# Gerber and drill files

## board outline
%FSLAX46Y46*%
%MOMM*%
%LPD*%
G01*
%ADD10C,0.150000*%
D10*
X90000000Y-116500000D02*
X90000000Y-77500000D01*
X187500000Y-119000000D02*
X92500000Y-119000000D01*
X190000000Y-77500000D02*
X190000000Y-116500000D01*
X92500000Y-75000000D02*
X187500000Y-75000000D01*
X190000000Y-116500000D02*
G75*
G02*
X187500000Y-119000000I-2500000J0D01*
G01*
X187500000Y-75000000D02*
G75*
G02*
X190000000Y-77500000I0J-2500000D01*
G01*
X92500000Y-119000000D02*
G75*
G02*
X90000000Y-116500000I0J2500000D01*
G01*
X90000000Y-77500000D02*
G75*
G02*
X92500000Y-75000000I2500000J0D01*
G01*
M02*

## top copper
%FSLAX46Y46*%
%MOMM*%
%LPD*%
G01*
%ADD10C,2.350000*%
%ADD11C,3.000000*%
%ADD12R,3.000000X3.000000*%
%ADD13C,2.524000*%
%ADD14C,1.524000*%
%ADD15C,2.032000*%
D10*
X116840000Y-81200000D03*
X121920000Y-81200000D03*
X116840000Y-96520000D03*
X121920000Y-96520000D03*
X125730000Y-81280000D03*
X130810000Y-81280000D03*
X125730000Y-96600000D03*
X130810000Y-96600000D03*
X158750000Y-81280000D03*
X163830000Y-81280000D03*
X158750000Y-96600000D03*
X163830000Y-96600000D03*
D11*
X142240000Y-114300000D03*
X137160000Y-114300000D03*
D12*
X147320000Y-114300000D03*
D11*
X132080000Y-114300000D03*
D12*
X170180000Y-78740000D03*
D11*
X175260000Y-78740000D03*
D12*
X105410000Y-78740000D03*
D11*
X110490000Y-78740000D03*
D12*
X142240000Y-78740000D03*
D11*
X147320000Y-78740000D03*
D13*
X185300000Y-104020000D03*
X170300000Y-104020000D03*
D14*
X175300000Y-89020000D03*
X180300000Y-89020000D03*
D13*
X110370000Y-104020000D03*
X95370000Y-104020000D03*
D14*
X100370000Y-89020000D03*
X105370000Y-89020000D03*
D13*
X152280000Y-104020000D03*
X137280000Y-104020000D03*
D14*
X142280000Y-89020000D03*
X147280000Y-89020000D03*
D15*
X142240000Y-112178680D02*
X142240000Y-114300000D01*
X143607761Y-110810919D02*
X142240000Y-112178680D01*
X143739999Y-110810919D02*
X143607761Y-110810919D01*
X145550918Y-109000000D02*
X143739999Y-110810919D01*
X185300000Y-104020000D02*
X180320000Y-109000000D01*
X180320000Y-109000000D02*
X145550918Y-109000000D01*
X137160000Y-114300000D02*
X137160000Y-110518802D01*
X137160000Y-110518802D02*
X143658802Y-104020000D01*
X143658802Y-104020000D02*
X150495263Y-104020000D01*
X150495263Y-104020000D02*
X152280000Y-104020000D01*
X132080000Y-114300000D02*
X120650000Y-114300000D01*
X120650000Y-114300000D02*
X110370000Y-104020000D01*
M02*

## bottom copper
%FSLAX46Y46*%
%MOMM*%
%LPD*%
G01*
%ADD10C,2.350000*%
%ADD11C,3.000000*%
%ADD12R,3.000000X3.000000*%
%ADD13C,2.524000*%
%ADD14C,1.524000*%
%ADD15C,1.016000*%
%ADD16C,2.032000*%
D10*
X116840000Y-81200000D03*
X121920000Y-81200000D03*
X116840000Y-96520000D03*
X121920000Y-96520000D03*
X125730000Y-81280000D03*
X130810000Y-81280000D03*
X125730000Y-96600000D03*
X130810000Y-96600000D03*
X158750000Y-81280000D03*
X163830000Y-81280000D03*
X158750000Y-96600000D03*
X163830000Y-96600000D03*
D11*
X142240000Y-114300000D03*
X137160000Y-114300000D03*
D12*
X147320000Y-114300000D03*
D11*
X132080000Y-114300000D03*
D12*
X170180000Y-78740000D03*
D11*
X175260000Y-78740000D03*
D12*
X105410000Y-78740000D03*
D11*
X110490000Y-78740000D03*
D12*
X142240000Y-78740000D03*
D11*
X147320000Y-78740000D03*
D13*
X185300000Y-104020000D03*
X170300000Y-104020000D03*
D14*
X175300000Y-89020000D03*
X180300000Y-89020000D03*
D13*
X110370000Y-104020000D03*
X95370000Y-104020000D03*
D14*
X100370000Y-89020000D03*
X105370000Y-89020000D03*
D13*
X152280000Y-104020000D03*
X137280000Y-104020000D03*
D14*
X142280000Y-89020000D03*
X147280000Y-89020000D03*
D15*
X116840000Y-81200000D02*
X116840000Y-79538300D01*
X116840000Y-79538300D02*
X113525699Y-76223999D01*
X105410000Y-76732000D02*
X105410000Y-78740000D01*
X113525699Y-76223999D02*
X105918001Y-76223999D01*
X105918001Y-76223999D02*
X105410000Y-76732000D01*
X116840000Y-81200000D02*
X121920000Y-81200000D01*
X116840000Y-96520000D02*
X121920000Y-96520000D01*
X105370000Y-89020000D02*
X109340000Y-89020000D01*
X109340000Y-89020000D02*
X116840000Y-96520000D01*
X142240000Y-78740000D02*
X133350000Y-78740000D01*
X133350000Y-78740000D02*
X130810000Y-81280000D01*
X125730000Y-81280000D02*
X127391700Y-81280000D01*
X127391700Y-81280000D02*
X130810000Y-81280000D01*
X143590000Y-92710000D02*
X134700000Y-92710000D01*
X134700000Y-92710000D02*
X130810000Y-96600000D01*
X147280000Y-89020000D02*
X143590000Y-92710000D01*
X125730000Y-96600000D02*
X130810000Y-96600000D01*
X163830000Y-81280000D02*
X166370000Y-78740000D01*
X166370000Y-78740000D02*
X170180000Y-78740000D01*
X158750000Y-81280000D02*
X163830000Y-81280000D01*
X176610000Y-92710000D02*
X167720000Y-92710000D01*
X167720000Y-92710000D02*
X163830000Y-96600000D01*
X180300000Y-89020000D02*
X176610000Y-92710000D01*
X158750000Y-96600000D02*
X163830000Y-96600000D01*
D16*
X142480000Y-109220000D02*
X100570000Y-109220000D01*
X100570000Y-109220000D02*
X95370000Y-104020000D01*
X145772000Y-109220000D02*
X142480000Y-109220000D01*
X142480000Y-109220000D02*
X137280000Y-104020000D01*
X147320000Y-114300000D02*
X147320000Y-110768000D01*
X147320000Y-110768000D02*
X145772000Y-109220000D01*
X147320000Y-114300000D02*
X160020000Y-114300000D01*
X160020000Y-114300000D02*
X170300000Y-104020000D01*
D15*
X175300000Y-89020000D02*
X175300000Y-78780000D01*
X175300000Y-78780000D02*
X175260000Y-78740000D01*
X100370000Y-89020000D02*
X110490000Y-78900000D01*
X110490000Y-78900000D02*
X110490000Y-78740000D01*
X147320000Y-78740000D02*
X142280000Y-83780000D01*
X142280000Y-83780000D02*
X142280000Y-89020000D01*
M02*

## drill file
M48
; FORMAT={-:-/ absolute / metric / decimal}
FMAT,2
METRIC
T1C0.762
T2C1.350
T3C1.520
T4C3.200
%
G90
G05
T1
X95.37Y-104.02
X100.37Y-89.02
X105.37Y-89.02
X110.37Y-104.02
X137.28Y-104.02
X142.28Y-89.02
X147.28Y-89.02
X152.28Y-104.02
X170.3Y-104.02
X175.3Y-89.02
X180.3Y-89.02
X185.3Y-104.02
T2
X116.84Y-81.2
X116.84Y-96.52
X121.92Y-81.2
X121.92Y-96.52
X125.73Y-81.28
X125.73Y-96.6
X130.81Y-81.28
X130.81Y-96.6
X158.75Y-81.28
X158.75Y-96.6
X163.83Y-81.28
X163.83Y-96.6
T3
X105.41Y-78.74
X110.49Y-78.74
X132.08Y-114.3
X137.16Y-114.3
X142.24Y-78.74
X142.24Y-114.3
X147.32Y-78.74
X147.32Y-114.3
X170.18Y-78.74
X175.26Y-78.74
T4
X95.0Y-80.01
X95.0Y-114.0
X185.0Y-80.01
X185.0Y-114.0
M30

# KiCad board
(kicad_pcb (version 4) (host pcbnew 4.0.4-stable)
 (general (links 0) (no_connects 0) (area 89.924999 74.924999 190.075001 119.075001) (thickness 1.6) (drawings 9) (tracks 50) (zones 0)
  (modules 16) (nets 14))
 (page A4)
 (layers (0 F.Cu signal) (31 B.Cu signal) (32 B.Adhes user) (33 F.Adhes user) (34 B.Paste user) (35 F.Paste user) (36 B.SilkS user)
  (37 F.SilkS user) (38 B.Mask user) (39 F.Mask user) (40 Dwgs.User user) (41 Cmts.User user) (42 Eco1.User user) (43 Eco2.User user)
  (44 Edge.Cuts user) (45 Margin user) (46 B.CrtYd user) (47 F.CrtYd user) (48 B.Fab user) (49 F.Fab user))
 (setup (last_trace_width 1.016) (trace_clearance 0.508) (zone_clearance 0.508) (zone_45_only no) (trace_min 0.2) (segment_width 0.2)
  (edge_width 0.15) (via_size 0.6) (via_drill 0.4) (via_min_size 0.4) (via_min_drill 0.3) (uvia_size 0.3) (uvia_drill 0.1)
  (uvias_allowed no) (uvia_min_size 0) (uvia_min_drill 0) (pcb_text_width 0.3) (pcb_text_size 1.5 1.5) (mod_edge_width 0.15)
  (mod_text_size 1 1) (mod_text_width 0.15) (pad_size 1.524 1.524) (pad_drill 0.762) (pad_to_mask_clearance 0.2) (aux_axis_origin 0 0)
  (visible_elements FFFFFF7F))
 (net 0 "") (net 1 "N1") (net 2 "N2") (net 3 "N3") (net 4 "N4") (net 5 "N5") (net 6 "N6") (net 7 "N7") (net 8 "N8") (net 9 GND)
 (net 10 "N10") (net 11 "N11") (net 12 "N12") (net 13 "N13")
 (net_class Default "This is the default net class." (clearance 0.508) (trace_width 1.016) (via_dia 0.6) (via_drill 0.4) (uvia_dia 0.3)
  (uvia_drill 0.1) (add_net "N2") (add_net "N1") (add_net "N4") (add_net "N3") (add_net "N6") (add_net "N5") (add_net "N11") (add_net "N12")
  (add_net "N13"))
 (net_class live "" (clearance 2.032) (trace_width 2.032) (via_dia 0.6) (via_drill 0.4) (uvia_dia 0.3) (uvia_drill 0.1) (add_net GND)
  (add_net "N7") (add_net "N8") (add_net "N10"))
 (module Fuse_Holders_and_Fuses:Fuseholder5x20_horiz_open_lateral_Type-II (layer F.Cu) (at 116.84 96.52 90)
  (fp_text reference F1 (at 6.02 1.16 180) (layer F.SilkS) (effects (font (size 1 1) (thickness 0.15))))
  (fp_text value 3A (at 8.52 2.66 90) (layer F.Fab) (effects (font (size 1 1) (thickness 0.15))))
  (pad 2 thru_hole circle (at 15.32 0 90) (size 2.35 2.35) (drill 1.35) (layers *.Cu *.Mask) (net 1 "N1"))
  (pad 2 thru_hole circle (at 15.32 5.08 90) (size 2.35 2.35) (drill 1.35) (layers *.Cu *.Mask) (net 1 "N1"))
  (pad 1 thru_hole circle (at 0 0 90) (size 2.35 2.35) (drill 1.35) (layers *.Cu *.Mask) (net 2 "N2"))
  (pad 1 thru_hole circle (at 0 5.08 90) (size 2.35 2.35) (drill 1.35) (layers *.Cu *.Mask) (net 2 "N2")))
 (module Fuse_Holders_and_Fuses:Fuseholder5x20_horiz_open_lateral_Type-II (layer F.Cu) (at 125.73 96.6 90)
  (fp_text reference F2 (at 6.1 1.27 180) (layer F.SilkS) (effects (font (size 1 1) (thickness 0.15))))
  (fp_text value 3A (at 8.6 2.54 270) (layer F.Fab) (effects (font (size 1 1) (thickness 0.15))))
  (pad 2 thru_hole circle (at 15.32 0 90) (size 2.35 2.35) (drill 1.35) (layers *.Cu *.Mask) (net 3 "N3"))
  (pad 2 thru_hole circle (at 15.32 5.08 90) (size 2.35 2.35) (drill 1.35) (layers *.Cu *.Mask) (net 3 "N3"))
  (pad 1 thru_hole circle (at 0 0 90) (size 2.35 2.35) (drill 1.35) (layers *.Cu *.Mask) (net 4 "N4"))
  (pad 1 thru_hole circle (at 0 5.08 90) (size 2.35 2.35) (drill 1.35) (layers *.Cu *.Mask) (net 4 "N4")))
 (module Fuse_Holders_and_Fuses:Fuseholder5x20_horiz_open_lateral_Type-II (layer F.Cu) (at 158.75 96.6 90)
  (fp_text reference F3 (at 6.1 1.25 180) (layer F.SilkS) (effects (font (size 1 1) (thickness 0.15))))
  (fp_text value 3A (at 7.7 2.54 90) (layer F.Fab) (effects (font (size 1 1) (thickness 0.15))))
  (pad 2 thru_hole circle (at 15.32 0 90) (size 2.35 2.35) (drill 1.35) (layers *.Cu *.Mask) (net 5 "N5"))
  (pad 2 thru_hole circle (at 15.32 5.08 90) (size 2.35 2.35) (drill 1.35) (layers *.Cu *.Mask) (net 5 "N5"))
  (pad 1 thru_hole circle (at 0 0 90) (size 2.35 2.35) (drill 1.35) (layers *.Cu *.Mask) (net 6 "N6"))
  (pad 1 thru_hole circle (at 0 5.08 90) (size 2.35 2.35) (drill 1.35) (layers *.Cu *.Mask) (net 6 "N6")))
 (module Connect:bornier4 (layer F.Cu) (at 147.32 114.3 180)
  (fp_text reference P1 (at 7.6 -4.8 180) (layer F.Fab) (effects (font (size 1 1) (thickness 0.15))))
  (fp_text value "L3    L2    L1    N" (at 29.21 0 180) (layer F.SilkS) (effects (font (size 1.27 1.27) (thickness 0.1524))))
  (pad 2 thru_hole circle (at 5.08 0 180) (size 3 3) (drill 1.52) (layers *.Cu *.Mask) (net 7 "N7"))
  (pad 3 thru_hole circle (at 10.16 0 180) (size 3 3) (drill 1.52) (layers *.Cu *.Mask) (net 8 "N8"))
  (pad 1 thru_hole rect (at 0 0 180) (size 3 3) (drill 1.52) (layers *.Cu *.Mask) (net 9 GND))
  (pad 4 thru_hole circle (at 15.24 0 180) (size 3 3) (drill 1.52) (layers *.Cu *.Mask) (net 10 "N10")))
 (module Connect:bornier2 (layer F.Cu) (at 170.18 78.74)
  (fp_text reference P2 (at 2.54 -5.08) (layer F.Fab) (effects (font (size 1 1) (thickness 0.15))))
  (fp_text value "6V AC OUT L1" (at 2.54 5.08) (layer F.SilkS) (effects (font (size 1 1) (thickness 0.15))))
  (pad 1 thru_hole rect (at 0 0) (size 3 3) (drill 1.52) (layers *.Cu *.Mask) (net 5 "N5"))
  (pad 2 thru_hole circle (at 5.08 0) (size 3 3) (drill 1.52) (layers *.Cu *.Mask) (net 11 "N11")))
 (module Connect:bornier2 (layer F.Cu) (at 105.41 78.74)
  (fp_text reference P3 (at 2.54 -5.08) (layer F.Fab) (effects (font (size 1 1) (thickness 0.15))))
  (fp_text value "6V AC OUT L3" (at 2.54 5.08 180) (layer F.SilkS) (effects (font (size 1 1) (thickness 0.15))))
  (pad 1 thru_hole rect (at 0 0) (size 3 3) (drill 1.52) (layers *.Cu *.Mask) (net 1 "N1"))
  (pad 2 thru_hole circle (at 5.08 0) (size 3 3) (drill 1.52) (layers *.Cu *.Mask) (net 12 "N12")))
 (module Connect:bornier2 (layer F.Cu) (at 142.24 78.74)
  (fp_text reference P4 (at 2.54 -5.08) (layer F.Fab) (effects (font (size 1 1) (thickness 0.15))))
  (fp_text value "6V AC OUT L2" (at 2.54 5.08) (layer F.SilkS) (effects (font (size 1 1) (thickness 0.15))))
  (pad 1 thru_hole rect (at 0 0) (size 3 3) (drill 1.52) (layers *.Cu *.Mask) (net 3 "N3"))
  (pad 2 thru_hole circle (at 5.08 0) (size 3 3) (drill 1.52) (layers *.Cu *.Mask) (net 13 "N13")))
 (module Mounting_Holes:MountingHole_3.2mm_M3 (layer F.Cu) (at 185 80.01 90)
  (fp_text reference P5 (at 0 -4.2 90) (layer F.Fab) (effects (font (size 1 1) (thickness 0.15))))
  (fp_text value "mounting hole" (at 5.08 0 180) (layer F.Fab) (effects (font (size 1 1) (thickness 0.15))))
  (pad 1 np_thru_hole circle (at 0 0 90) (size 3.2 3.2) (drill 3.2) (layers *.Cu *.Mask)))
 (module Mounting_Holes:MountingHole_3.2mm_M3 (layer F.Cu) (at 185 114 90)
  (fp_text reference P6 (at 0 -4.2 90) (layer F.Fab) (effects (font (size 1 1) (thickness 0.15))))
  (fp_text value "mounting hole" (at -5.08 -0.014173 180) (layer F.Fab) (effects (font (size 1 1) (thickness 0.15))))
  (pad 1 np_thru_hole circle (at 0 0 90) (size 3.2 3.2) (drill 3.2) (layers *.Cu *.Mask)))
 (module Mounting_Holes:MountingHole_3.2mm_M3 (layer F.Cu) (at 95 114 90)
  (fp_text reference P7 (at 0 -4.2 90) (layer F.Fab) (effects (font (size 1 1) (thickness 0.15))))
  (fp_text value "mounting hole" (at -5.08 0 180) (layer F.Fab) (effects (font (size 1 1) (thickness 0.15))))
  (pad 1 np_thru_hole circle (at 0 0 90) (size 3.2 3.2) (drill 3.2) (layers *.Cu *.Mask)))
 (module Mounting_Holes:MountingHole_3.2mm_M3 (layer F.Cu) (at 95 80.01 90)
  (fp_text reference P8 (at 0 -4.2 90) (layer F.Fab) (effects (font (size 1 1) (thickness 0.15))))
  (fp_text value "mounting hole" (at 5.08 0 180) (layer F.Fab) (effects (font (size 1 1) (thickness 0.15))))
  (pad 1 np_thru_hole circle (at 0 0 90) (size 3.2 3.2) (drill 3.2) (layers *.Cu *.Mask)))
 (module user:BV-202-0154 (layer F.Cu) (at 177.8 96.52 90)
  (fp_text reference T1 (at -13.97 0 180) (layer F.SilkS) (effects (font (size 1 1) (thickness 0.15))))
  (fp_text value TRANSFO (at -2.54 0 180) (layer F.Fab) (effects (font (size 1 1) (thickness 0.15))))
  (pad 1 thru_hole circle (at -7.5 7.5 90) (size 2.524 2.524) (drill 0.762) (layers *.Cu *.Mask) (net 7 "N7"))
  (pad 2 thru_hole circle (at -7.5 -7.5 90) (size 2.524 2.524) (drill 0.762) (layers *.Cu *.Mask) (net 9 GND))
  (pad 3 thru_hole circle (at 7.5 -2.5 90) (size 1.524 1.524) (drill 0.762) (layers *.Cu *.Mask) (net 11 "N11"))
  (pad 4 thru_hole circle (at 7.5 2.5 90) (size 1.524 1.524) (drill 0.762) (layers *.Cu *.Mask) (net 6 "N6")))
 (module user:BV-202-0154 (layer F.Cu) (at 102.87 96.52 90)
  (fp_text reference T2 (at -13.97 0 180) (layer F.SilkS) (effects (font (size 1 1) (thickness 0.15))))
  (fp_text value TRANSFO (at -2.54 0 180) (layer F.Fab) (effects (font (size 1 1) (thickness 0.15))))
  (pad 1 thru_hole circle (at -7.5 7.5 90) (size 2.524 2.524) (drill 0.762) (layers *.Cu *.Mask) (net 10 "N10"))
  (pad 2 thru_hole circle (at -7.5 -7.5 90) (size 2.524 2.524) (drill 0.762) (layers *.Cu *.Mask) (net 9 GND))
  (pad 3 thru_hole circle (at 7.5 -2.5 90) (size 1.524 1.524) (drill 0.762) (layers *.Cu *.Mask) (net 12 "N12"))
  (pad 4 thru_hole circle (at 7.5 2.5 90) (size 1.524 1.524) (drill 0.762) (layers *.Cu *.Mask) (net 2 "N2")))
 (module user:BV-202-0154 (layer F.Cu) (at 144.78 96.52 90)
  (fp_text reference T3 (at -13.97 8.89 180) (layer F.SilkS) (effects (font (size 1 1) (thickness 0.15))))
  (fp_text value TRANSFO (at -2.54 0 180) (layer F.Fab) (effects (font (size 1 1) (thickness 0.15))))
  (pad 1 thru_hole circle (at -7.5 7.5 90) (size 2.524 2.524) (drill 0.762) (layers *.Cu *.Mask) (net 8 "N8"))
  (pad 2 thru_hole circle (at -7.5 -7.5 90) (size 2.524 2.524) (drill 0.762) (layers *.Cu *.Mask) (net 9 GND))
  (pad 3 thru_hole circle (at 7.5 -2.5 90) (size 1.524 1.524) (drill 0.762) (layers *.Cu *.Mask) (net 13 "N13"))
  (pad 4 thru_hole circle (at 7.5 2.5 90) (size 1.524 1.524) (drill 0.762) (layers *.Cu *.Mask) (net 4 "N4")))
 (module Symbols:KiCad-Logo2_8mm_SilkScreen (layer F.Cu) (at 124 106)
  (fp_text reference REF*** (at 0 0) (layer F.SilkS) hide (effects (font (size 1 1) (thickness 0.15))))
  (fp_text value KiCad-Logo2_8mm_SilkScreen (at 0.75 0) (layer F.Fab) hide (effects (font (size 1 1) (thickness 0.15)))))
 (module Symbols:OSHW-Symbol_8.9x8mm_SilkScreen (layer F.Cu) (at 161 109.5)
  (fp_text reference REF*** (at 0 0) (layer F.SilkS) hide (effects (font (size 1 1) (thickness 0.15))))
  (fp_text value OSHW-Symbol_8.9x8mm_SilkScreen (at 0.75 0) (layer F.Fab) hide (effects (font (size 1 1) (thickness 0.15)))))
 (gr_line (start 90 116.5) (end 90 77.5) (layer Edge.Cuts) (width 0.15))
 (gr_line (start 187.5 119) (end 92.5 119) (layer Edge.Cuts) (width 0.15))
 (gr_line (start 190 77.5) (end 190 116.5) (layer Edge.Cuts) (width 0.15))
 (gr_line (start 92.5 75) (end 187.5 75) (layer Edge.Cuts) (width 0.15))
 (gr_arc (start 187.5 116.5) (end 190 116.5) (angle 90) (layer Edge.Cuts) (width 0.15))
 (gr_arc (start 187.5 77.5) (end 187.5 75) (angle 90) (layer Edge.Cuts) (width 0.15))
 (gr_arc (start 92.5 116.5) (end 92.5 119) (angle 90) (layer Edge.Cuts) (width 0.15))
 (gr_arc (start 92.5 77.5) (end 90 77.5) (angle 90) (layer Edge.Cuts) (width 0.15))
 (segment (start 116.84 81.2) (end 116.84 79.5383) (width 1.016) (layer B.Cu) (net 1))
 (segment (start 116.84 79.5383) (end 113.525699 76.223999) (width 1.016) (layer B.Cu) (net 1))
 (segment (start 105.41 76.732) (end 105.41 78.74) (width 1.016) (layer B.Cu) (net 1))
 (segment (start 113.525699 76.223999) (end 105.918001 76.223999) (width 1.016) (layer B.Cu) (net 1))
 (segment (start 105.918001 76.223999) (end 105.41 76.732) (width 1.016) (layer B.Cu) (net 1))
 (segment (start 116.84 81.2) (end 121.92 81.2) (width 1.016) (layer B.Cu) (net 1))
 (segment (start 116.84 96.52) (end 121.92 96.52) (width 1.016) (layer B.Cu) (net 2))
 (segment (start 105.37 89.02) (end 109.34 89.02) (width 1.016) (layer B.Cu) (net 2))
 (segment (start 109.34 89.02) (end 116.84 96.52) (width 1.016) (layer B.Cu) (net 2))
 (segment (start 142.24 78.74) (end 133.35 78.74) (width 1.016) (layer B.Cu) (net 3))
 (segment (start 133.35 78.74) (end 130.81 81.28) (width 1.016) (layer B.Cu) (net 3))
 (segment (start 125.73 81.28) (end 127.3917 81.28) (width 1.016) (layer B.Cu) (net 3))
 (segment (start 127.3917 81.28) (end 130.81 81.28) (width 1.016) (layer B.Cu) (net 3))
 (segment (start 143.59 92.71) (end 134.7 92.71) (width 1.016) (layer B.Cu) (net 4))
 (segment (start 134.7 92.71) (end 130.81 96.6) (width 1.016) (layer B.Cu) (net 4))
 (segment (start 147.28 89.02) (end 143.59 92.71) (width 1.016) (layer B.Cu) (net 4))
 (segment (start 125.73 96.6) (end 130.81 96.6) (width 1.016) (layer B.Cu) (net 4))
 (segment (start 163.83 81.28) (end 166.37 78.74) (width 1.016) (layer B.Cu) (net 5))
 (segment (start 166.37 78.74) (end 170.18 78.74) (width 1.016) (layer B.Cu) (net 5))
 (segment (start 158.75 81.28) (end 163.83 81.28) (width 1.016) (layer B.Cu) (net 5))
 (segment (start 176.61 92.71) (end 167.72 92.71) (width 1.016) (layer B.Cu) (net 6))
 (segment (start 167.72 92.71) (end 163.83 96.6) (width 1.016) (layer B.Cu) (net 6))
 (segment (start 180.3 89.02) (end 176.61 92.71) (width 1.016) (layer B.Cu) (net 6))
 (segment (start 158.75 96.6) (end 163.83 96.6) (width 1.016) (layer B.Cu) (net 6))
 (segment (start 142.24 112.17868) (end 142.24 114.3) (width 2.032) (layer F.Cu) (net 7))
 (segment (start 143.607761 110.810919) (end 142.24 112.17868) (width 2.032) (layer F.Cu) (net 7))
 (segment (start 143.739999 110.810919) (end 143.607761 110.810919) (width 2.032) (layer F.Cu) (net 7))
 (segment (start 145.550918 109) (end 143.739999 110.810919) (width 2.032) (layer F.Cu) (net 7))
 (segment (start 185.3 104.02) (end 180.32 109) (width 2.032) (layer F.Cu) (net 7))
 (segment (start 180.32 109) (end 145.550918 109) (width 2.032) (layer F.Cu) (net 7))
 (segment (start 137.16 114.3) (end 137.16 110.518802) (width 2.032) (layer F.Cu) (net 8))
 (segment (start 137.16 110.518802) (end 143.658802 104.02) (width 2.032) (layer F.Cu) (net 8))
 (segment (start 143.658802 104.02) (end 150.495263 104.02) (width 2.032) (layer F.Cu) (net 8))
 (segment (start 150.495263 104.02) (end 152.28 104.02) (width 2.032) (layer F.Cu) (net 8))
 (segment (start 142.48 109.22) (end 100.57 109.22) (width 2.032) (layer B.Cu) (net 9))
 (segment (start 100.57 109.22) (end 95.37 104.02) (width 2.032) (layer B.Cu) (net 9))
 (segment (start 145.772 109.22) (end 142.48 109.22) (width 2.032) (layer B.Cu) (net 9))
 (segment (start 142.48 109.22) (end 137.28 104.02) (width 2.032) (layer B.Cu) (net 9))
 (segment (start 147.32 114.3) (end 147.32 110.768) (width 2.032) (layer B.Cu) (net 9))
 (segment (start 147.32 110.768) (end 145.772 109.22) (width 2.032) (layer B.Cu) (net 9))
 (segment (start 147.32 114.3) (end 160.02 114.3) (width 2.032) (layer B.Cu) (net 9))
 (segment (start 160.02 114.3) (end 170.3 104.02) (width 2.032) (layer B.Cu) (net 9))
 (segment (start 132.08 114.3) (end 120.65 114.3) (width 2.032) (layer F.Cu) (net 10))
 (segment (start 120.65 114.3) (end 110.37 104.02) (width 2.032) (layer F.Cu) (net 10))
 (segment (start 175.3 89.02) (end 175.3 78.78) (width 1.016) (layer B.Cu) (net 11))
 (segment (start 175.3 78.78) (end 175.26 78.74) (width 1.016) (layer B.Cu) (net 11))
 (segment (start 100.37 89.02) (end 110.49 78.9) (width 1.016) (layer B.Cu) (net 12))
 (segment (start 110.49 78.9) (end 110.49 78.74) (width 1.016) (layer B.Cu) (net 12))
 (segment (start 147.32 78.74) (end 142.28 83.78) (width 1.016) (layer B.Cu) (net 13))
 (segment (start 142.28 83.78) (end 142.28 89.02) (width 1.016) (layer B.Cu) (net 13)))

